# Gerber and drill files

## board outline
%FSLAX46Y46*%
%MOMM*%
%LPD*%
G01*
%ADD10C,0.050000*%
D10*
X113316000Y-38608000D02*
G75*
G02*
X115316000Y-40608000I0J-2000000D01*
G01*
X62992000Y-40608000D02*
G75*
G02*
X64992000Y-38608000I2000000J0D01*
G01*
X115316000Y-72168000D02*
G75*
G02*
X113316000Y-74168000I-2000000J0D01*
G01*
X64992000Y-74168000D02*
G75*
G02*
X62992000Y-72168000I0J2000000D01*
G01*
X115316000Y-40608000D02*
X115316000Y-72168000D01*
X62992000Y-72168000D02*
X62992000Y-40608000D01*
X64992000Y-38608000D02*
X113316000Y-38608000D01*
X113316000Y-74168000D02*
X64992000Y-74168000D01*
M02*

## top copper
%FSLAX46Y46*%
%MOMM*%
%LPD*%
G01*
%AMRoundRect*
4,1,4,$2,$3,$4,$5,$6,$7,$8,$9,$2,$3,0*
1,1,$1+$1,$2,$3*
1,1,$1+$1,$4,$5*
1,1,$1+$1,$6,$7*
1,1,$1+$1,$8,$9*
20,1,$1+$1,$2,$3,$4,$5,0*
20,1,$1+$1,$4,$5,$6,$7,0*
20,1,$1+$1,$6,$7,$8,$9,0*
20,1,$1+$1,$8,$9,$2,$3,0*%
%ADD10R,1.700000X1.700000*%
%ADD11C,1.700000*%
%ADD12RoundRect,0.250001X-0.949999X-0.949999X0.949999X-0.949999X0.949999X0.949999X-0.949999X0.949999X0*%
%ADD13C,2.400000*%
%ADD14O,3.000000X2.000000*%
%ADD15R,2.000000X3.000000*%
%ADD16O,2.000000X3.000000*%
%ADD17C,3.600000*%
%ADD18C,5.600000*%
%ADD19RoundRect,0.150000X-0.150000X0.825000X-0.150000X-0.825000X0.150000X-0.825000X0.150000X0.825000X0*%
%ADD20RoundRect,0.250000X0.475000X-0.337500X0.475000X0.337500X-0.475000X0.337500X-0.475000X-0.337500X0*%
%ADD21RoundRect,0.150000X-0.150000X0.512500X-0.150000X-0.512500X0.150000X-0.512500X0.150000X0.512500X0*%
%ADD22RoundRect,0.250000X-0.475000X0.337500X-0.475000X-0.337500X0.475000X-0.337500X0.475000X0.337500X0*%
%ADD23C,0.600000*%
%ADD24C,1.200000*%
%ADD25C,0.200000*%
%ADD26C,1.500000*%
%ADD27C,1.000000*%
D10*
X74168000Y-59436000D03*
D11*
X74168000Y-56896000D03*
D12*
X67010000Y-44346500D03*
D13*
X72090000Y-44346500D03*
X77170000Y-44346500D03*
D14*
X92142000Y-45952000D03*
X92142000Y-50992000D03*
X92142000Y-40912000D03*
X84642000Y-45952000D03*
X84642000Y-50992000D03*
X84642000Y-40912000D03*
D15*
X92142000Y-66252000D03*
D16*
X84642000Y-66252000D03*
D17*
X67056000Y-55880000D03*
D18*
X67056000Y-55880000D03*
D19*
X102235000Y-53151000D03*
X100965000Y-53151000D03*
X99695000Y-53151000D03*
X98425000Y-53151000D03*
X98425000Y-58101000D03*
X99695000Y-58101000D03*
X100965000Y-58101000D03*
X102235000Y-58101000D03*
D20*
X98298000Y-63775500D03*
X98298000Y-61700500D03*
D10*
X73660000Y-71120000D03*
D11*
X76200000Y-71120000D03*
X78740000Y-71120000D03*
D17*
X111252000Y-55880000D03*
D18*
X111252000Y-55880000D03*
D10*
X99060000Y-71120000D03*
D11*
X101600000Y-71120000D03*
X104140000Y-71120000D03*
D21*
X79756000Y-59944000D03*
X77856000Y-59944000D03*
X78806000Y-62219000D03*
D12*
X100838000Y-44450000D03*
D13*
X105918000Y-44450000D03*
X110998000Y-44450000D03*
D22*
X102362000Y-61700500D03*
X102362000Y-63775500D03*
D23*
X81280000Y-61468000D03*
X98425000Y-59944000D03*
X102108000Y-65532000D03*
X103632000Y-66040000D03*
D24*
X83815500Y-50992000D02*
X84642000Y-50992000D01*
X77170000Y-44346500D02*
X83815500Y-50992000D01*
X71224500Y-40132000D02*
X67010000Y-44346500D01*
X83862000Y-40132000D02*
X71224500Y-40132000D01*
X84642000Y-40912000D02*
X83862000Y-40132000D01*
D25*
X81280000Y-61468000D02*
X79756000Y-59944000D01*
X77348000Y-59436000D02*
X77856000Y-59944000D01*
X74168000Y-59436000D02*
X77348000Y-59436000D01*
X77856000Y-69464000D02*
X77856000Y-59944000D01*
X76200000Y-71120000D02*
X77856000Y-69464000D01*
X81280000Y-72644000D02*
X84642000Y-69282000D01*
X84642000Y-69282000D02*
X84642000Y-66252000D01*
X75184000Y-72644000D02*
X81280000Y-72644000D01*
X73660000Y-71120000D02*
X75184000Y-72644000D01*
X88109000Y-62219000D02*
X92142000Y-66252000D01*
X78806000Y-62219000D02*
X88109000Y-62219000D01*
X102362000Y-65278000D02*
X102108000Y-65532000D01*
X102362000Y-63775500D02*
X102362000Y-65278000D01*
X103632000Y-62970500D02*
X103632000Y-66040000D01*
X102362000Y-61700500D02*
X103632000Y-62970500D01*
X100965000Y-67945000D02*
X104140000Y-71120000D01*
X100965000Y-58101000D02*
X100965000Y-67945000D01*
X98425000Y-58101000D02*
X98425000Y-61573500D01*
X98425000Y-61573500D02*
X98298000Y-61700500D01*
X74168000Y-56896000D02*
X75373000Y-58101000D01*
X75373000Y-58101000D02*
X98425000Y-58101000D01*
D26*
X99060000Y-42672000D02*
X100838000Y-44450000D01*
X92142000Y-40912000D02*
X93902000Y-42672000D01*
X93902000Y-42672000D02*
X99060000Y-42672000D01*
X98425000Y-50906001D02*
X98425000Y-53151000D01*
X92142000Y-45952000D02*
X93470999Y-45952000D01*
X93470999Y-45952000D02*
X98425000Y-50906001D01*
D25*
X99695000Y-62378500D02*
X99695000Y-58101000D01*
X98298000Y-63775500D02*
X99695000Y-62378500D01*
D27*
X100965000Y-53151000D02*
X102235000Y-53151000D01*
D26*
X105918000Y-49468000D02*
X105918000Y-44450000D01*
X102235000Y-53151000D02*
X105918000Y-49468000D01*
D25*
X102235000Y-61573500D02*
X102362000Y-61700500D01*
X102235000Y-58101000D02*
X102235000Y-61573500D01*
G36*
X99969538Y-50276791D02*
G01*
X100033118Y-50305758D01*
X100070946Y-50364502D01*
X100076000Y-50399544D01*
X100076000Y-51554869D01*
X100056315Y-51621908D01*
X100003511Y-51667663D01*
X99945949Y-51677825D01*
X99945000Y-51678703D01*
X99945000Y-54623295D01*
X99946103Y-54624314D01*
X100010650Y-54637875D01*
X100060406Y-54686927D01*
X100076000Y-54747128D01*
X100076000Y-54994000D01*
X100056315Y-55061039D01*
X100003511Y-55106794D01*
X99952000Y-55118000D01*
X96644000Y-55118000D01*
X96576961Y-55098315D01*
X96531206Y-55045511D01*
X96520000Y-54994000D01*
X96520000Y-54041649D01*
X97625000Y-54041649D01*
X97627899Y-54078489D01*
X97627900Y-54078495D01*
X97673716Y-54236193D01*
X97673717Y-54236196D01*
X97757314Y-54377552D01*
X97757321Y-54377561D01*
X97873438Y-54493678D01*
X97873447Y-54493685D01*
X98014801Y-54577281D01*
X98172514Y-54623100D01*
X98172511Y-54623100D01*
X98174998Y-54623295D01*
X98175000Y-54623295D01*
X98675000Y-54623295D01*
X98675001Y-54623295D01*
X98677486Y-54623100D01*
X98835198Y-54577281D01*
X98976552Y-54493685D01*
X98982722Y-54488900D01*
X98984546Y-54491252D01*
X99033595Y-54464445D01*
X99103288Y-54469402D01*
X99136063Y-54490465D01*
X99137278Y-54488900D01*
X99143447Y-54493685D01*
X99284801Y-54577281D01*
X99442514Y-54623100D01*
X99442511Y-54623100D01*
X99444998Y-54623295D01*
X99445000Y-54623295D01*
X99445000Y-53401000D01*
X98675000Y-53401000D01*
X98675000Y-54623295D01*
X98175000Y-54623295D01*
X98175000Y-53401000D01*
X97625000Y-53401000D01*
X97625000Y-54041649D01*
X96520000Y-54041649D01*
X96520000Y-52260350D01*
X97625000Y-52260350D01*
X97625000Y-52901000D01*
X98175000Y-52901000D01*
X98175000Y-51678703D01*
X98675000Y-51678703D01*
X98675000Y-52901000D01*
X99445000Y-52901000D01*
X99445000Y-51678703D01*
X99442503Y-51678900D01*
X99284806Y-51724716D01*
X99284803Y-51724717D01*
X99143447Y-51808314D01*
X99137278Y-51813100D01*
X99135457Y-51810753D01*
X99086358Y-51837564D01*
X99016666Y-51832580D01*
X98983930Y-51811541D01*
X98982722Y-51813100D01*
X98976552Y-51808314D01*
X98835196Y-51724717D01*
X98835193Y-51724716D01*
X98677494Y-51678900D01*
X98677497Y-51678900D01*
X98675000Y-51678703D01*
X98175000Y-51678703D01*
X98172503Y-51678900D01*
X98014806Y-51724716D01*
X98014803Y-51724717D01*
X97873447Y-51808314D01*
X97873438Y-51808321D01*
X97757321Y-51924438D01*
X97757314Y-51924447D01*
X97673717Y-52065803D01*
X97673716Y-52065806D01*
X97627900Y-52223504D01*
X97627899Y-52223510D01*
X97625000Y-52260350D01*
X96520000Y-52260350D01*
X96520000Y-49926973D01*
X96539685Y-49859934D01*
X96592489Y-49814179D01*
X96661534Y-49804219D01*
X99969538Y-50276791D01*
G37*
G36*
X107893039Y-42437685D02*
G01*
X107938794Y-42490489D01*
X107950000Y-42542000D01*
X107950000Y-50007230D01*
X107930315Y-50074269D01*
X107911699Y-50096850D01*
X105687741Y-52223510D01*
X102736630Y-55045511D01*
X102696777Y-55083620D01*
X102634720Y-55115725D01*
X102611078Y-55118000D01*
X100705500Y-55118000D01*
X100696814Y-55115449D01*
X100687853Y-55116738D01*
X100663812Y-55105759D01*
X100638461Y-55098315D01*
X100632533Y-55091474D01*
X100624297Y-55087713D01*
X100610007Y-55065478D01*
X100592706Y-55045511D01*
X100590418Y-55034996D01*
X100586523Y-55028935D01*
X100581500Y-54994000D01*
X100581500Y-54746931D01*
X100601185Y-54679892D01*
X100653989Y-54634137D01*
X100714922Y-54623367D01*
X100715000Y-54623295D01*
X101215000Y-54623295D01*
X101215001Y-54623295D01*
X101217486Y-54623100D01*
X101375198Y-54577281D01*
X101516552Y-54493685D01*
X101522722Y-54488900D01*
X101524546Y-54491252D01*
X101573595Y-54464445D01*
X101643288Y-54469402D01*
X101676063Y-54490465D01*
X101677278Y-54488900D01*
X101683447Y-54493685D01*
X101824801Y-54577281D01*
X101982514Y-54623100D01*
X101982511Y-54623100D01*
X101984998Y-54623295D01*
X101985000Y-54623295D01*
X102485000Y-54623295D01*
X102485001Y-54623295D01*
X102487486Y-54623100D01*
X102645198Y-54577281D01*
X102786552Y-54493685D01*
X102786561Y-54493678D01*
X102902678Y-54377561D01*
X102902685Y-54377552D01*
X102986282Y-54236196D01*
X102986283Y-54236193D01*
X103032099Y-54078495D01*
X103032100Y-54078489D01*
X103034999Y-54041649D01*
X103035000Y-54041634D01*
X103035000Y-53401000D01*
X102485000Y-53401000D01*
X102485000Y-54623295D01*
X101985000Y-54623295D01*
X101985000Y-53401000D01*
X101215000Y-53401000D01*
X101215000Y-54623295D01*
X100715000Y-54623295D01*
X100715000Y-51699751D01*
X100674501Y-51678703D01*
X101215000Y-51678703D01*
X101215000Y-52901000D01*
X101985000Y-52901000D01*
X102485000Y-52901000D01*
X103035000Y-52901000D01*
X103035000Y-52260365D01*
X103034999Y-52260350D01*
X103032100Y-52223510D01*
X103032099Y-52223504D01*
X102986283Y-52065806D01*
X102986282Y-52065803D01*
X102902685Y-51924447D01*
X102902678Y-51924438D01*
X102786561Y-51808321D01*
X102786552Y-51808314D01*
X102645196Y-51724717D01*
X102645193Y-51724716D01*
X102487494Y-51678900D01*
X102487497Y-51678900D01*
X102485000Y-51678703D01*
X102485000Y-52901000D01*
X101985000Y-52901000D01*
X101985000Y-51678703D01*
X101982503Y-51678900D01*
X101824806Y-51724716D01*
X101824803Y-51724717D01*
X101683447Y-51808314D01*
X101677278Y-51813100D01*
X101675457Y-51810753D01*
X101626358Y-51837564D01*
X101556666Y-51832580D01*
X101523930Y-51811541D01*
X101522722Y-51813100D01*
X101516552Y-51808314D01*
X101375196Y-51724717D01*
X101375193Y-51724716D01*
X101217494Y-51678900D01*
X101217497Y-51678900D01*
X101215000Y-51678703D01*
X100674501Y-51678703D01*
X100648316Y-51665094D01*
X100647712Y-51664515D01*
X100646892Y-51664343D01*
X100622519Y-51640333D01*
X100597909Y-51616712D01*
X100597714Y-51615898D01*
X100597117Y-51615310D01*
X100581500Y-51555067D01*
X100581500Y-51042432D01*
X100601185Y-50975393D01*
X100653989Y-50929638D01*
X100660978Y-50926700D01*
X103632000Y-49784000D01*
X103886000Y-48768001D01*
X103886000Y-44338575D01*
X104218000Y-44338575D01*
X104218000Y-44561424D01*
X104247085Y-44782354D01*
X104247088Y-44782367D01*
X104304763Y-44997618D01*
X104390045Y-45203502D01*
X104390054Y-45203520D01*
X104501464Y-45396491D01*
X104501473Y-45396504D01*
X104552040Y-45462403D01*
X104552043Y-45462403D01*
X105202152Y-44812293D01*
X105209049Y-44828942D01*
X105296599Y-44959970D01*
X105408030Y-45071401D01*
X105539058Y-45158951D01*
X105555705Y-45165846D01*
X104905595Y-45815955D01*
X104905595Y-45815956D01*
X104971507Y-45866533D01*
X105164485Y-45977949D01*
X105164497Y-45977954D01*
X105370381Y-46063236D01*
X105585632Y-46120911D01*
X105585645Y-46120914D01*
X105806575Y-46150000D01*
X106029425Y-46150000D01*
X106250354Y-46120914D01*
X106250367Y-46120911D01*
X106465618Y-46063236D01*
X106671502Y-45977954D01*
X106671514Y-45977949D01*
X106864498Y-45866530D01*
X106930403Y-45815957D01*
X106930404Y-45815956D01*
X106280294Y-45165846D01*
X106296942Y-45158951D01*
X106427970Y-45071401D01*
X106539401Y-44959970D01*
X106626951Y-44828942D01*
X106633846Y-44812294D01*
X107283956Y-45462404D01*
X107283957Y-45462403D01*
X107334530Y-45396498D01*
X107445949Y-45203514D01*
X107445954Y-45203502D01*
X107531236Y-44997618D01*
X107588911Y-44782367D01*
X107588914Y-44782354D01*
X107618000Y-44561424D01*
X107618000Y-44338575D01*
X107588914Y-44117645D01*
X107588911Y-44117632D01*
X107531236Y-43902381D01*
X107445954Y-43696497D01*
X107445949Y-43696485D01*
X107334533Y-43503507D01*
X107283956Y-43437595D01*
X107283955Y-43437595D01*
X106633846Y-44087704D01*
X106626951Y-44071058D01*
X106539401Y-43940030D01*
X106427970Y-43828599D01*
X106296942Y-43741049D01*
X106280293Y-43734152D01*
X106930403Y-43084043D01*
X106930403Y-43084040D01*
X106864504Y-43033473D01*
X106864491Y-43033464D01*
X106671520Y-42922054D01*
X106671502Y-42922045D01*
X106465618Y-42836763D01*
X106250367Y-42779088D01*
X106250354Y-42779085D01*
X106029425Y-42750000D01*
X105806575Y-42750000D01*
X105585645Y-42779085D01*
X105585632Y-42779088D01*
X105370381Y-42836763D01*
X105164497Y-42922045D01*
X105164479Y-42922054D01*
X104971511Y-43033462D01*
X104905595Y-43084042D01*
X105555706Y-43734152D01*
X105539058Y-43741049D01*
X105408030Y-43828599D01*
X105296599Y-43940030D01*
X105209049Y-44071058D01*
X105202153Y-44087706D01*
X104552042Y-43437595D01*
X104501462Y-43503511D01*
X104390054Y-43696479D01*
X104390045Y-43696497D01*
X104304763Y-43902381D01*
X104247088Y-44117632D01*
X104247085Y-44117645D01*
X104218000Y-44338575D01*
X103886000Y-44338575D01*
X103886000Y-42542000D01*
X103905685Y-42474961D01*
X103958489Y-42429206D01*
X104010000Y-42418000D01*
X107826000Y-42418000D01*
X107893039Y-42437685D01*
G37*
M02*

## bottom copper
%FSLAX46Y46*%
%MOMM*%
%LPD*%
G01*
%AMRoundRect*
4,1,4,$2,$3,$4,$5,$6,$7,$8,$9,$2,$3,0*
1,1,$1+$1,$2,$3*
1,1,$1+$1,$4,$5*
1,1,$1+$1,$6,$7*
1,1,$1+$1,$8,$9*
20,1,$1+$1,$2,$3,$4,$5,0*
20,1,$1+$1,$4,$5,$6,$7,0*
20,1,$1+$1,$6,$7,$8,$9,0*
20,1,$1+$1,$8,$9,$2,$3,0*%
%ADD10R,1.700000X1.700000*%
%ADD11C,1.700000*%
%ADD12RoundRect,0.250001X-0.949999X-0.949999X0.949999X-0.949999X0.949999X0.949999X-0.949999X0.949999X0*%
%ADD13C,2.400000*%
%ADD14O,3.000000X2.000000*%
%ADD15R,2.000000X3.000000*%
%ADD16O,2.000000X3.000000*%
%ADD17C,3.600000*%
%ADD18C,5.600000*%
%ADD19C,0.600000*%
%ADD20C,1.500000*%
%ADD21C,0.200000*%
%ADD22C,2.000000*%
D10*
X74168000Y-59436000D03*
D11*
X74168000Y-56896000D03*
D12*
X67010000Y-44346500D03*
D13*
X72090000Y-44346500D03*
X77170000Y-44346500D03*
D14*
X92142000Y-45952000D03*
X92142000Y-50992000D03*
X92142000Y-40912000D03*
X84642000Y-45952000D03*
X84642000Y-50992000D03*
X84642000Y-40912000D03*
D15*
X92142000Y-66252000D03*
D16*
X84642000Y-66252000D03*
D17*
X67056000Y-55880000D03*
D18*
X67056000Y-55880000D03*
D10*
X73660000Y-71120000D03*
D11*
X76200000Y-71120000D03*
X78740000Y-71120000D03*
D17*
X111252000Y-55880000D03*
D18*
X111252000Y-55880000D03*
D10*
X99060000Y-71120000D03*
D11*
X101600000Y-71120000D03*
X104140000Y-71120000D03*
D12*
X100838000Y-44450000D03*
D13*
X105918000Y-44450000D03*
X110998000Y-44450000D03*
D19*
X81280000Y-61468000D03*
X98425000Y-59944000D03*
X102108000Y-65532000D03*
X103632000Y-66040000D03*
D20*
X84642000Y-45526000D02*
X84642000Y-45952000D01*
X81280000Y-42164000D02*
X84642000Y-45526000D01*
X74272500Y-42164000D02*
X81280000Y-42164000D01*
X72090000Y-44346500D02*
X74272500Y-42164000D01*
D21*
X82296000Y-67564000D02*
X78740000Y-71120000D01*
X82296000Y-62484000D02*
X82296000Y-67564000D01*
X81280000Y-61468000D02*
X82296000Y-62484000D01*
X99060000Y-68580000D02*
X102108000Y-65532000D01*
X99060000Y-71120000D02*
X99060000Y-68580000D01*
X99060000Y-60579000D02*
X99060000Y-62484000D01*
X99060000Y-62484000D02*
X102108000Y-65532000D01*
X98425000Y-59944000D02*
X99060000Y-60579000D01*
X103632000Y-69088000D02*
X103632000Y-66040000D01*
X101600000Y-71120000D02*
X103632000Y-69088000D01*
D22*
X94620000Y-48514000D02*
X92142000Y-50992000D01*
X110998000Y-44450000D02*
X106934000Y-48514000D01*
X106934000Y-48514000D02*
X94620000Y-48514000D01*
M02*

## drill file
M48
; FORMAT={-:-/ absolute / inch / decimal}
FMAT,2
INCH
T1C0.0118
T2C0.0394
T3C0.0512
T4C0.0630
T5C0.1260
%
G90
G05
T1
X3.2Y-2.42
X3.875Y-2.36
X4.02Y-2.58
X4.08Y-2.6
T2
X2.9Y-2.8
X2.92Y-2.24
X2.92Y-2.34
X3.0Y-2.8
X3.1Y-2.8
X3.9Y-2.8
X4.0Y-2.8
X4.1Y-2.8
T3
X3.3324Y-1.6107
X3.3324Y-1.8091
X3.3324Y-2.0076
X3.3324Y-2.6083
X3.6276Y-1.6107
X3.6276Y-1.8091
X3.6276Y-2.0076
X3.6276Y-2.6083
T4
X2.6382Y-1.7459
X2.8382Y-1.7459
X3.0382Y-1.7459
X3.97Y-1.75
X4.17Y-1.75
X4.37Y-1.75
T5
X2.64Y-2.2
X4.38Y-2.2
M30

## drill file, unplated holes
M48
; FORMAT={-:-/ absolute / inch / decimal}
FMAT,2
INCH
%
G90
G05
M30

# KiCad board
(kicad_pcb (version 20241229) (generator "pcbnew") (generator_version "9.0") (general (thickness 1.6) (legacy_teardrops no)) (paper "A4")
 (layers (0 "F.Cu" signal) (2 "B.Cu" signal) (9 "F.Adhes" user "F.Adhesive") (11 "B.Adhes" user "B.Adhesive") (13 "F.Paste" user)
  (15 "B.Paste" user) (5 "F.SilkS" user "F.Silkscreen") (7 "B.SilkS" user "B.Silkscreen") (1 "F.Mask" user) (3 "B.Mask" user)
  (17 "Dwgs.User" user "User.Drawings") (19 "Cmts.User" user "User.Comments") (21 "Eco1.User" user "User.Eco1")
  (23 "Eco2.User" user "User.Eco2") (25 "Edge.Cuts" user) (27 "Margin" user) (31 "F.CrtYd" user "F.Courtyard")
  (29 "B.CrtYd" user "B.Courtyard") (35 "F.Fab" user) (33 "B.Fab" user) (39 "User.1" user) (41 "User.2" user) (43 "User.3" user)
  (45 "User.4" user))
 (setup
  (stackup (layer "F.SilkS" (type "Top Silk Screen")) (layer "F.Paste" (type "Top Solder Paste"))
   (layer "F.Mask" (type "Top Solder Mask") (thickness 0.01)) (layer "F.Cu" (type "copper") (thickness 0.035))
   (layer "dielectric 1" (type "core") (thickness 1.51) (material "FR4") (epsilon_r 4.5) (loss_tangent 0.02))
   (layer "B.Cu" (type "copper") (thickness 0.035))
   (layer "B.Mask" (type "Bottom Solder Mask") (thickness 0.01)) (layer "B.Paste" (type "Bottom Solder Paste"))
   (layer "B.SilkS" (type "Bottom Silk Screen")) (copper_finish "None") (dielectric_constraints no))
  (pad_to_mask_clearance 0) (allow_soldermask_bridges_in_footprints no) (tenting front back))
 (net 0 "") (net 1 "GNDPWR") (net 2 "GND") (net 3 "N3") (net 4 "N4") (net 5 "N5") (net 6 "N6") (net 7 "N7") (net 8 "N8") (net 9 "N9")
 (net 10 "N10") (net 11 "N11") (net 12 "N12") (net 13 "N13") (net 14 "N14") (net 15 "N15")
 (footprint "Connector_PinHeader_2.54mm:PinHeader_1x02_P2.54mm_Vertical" (layer "F.Cu") (at 74.168 59.436 180)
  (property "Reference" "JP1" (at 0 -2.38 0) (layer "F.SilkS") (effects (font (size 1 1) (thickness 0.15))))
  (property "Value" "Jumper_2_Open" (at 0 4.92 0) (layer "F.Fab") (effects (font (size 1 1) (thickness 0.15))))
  (pad "1" thru_hole rect (at 0 0 180) (size 1.7 1.7) (drill 1) (layers "*.Cu" "*.Mask") (remove_unused_layers no) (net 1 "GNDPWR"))
  (pad "2" thru_hole circle (at 0 2.54 180) (size 1.7 1.7) (drill 1) (layers "*.Cu" "*.Mask") (remove_unused_layers no) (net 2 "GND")))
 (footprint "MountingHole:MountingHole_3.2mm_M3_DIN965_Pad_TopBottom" (layer "F.Cu") (at 67.056 55.88)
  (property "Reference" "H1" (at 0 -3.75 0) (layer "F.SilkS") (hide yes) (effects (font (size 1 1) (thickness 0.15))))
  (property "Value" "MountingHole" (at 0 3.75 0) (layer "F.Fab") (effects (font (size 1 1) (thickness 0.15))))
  (pad "1" thru_hole circle (at 0 0) (size 3.6 3.6) (drill 3.2) (layers "*.Cu" "*.Mask") (remove_unused_layers no) (zone_connect 2))
  (pad "1" connect circle (at 0 0) (size 5.6 5.6) (layers "F.Cu" "F.Mask") (zone_connect 2))
  (pad "1" connect circle (at 0 0) (size 5.6 5.6) (layers "B.Cu" "B.Mask") (zone_connect 2)))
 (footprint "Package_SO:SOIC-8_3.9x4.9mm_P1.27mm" (layer "F.Cu") (at 100.33 55.626 -90)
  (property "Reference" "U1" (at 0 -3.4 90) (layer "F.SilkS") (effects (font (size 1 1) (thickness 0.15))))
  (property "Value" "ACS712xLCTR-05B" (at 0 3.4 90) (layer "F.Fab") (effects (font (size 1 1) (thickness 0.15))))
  (pad "1" smd roundrect (at -2.475 -1.905 270) (size 1.95 0.6) (layers "F.Cu" "F.Mask" "F.Paste") (roundrect_rratio 0.25) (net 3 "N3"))
  (pad "2" smd roundrect (at -2.475 -0.635 270) (size 1.95 0.6) (layers "F.Cu" "F.Mask" "F.Paste") (roundrect_rratio 0.25) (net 3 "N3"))
  (pad "3" smd roundrect (at -2.475 0.635 270) (size 1.95 0.6) (layers "F.Cu" "F.Mask" "F.Paste") (roundrect_rratio 0.25) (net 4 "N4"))
  (pad "4" smd roundrect (at -2.475 1.905 270) (size 1.95 0.6) (layers "F.Cu" "F.Mask" "F.Paste") (roundrect_rratio 0.25) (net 4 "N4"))
  (pad "5" smd roundrect (at 2.475 1.905 270) (size 1.95 0.6) (layers "F.Cu" "F.Mask" "F.Paste") (roundrect_rratio 0.25) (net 2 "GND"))
  (pad "6" smd roundrect (at 2.475 0.635 270) (size 1.95 0.6) (layers "F.Cu" "F.Mask" "F.Paste") (roundrect_rratio 0.25) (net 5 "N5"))
  (pad "7" smd roundrect (at 2.475 -0.635 270) (size 1.95 0.6) (layers "F.Cu" "F.Mask" "F.Paste") (roundrect_rratio 0.25) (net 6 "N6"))
  (pad "8" smd roundrect (at 2.475 -1.905 270) (size 1.95 0.6) (layers "F.Cu" "F.Mask" "F.Paste") (roundrect_rratio 0.25) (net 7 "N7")))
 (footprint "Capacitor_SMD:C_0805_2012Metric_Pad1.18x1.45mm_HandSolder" (layer "F.Cu") (at 98.298 62.738 90)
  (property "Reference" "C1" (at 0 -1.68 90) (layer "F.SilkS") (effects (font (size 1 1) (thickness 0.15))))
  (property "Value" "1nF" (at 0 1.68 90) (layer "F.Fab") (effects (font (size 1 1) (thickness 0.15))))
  (pad "1" smd roundrect (at -1.0375 0 90) (size 1.175 1.45) (layers "F.Cu" "F.Mask" "F.Paste") (roundrect_rratio 0.212766) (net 5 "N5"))
  (pad "2" smd roundrect (at 1.0375 0 90) (size 1.175 1.45) (layers "F.Cu" "F.Mask" "F.Paste") (roundrect_rratio 0.212766) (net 2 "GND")))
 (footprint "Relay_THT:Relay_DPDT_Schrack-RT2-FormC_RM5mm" (layer "F.Cu") (at 92.142 66.252 90)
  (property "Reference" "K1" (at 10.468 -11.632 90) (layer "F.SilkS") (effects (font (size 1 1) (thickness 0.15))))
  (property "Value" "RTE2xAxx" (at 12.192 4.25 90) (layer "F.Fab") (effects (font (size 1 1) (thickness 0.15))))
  (pad "11" thru_hole oval (at 20.3 0 270) (size 2 3) (drill 1.3) (layers "*.Cu" "*.Mask") (remove_unused_layers no) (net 4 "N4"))
  (pad "12" thru_hole oval (at 15.26 0 270) (size 2 3) (drill 1.3) (layers "*.Cu" "*.Mask") (remove_unused_layers no) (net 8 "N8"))
  (pad "14" thru_hole oval (at 25.34 0 270) (size 2 3) (drill 1.3) (layers "*.Cu" "*.Mask") (remove_unused_layers no) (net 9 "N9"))
  (pad "21" thru_hole oval (at 20.3 -7.5 270) (size 2 3) (drill 1.3) (layers "*.Cu" "*.Mask") (remove_unused_layers no) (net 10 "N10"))
  (pad "22" thru_hole oval (at 15.26 -7.5 270) (size 2 3) (drill 1.3) (layers "*.Cu" "*.Mask") (remove_unused_layers no) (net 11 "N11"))
  (pad "24" thru_hole oval (at 25.34 -7.5 270) (size 2 3) (drill 1.3) (layers "*.Cu" "*.Mask") (remove_unused_layers no) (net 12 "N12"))
  (pad "A1" thru_hole rect (at 0 0 270) (size 3 2) (drill 1.3) (layers "*.Cu" "*.Mask") (remove_unused_layers no) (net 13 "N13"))
  (pad "A2" thru_hole oval (at 0 -7.5 270) (size 3 2) (drill 1.3) (layers "*.Cu" "*.Mask") (remove_unused_layers no) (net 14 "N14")))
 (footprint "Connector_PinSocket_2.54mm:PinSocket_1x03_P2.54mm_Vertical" (layer "F.Cu") (at 73.66 71.12 90)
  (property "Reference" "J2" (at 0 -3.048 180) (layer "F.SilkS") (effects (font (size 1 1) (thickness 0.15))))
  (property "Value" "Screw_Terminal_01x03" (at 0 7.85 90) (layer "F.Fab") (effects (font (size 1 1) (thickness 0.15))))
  (pad "1" thru_hole rect (at 0 0 90) (size 1.7 1.7) (drill 1) (layers "*.Cu" "*.Mask") (remove_unused_layers no) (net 14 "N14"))
  (pad "2" thru_hole circle (at 0 2.54 90) (size 1.7 1.7) (drill 1) (layers "*.Cu" "*.Mask") (remove_unused_layers no) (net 1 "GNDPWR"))
  (pad "3" thru_hole circle (at 0 5.08 90) (size 1.7 1.7) (drill 1) (layers "*.Cu" "*.Mask") (remove_unused_layers no) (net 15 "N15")))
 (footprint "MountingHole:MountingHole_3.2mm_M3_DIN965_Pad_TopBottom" (layer "F.Cu") (at 111.252 55.88)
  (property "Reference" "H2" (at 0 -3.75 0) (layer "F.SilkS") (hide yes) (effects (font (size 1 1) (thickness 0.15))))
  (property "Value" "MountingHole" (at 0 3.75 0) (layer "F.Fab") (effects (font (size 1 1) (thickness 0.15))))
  (pad "1" thru_hole circle (at 0 0) (size 3.6 3.6) (drill 3.2) (layers "*.Cu" "*.Mask") (remove_unused_layers no) (zone_connect 2))
  (pad "1" connect circle (at 0 0) (size 5.6 5.6) (layers "F.Cu" "F.Mask") (zone_connect 2))
  (pad "1" connect circle (at 0 0) (size 5.6 5.6) (layers "B.Cu" "B.Mask") (zone_connect 2)))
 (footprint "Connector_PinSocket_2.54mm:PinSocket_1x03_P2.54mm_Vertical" (layer "F.Cu") (at 99.06 71.12 90)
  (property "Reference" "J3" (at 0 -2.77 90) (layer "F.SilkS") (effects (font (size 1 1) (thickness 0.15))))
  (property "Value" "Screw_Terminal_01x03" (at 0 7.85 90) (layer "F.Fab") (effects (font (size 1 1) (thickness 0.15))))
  (pad "1" thru_hole rect (at 0 0 90) (size 1.7 1.7) (drill 1) (layers "*.Cu" "*.Mask") (remove_unused_layers no) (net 2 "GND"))
  (pad "2" thru_hole circle (at 0 2.54 90) (size 1.7 1.7) (drill 1) (layers "*.Cu" "*.Mask") (remove_unused_layers no) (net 7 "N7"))
  (pad "3" thru_hole circle (at 0 5.08 90) (size 1.7 1.7) (drill 1) (layers "*.Cu" "*.Mask") (remove_unused_layers no) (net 6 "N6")))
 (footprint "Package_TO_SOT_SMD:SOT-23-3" (layer "F.Cu") (at 78.806 61.0815 -90)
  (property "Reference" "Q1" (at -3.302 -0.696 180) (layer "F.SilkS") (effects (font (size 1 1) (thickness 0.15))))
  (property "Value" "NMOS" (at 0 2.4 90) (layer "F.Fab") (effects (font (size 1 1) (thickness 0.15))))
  (pad "1" smd roundrect (at -1.1375 -0.95 270) (size 1.325 0.6) (layers "F.Cu" "F.Mask" "F.Paste") (roundrect_rratio 0.25) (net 15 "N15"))
  (pad "2" smd roundrect (at -1.1375 0.95 270) (size 1.325 0.6) (layers "F.Cu" "F.Mask" "F.Paste") (roundrect_rratio 0.25) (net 1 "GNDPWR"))
  (pad "3" smd roundrect (at 1.1375 0 270) (size 1.325 0.6) (layers "F.Cu" "F.Mask" "F.Paste") (roundrect_rratio 0.25) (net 13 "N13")))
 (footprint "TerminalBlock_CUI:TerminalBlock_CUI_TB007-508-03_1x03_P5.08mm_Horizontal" (layer "F.Cu") (at 67.01 44.3465)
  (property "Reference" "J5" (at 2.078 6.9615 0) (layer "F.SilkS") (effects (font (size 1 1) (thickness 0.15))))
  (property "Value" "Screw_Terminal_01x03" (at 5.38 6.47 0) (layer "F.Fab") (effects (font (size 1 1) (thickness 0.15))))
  (pad "1" thru_hole roundrect (at 0 0) (size 2.4 2.4) (drill 1.6) (layers "*.Cu" "*.Mask") (remove_unused_layers no)
   (roundrect_rratio 0.104167) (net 12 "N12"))
  (pad "2" thru_hole circle (at 5.08 0) (size 2.4 2.4) (drill 1.6) (layers "*.Cu" "*.Mask") (remove_unused_layers no) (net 10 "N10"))
  (pad "3" thru_hole circle (at 10.16 0) (size 2.4 2.4) (drill 1.6) (layers "*.Cu" "*.Mask") (remove_unused_layers no) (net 11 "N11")))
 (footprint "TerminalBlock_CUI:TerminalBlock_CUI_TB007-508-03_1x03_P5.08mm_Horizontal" (layer "F.Cu") (at 100.838 44.45)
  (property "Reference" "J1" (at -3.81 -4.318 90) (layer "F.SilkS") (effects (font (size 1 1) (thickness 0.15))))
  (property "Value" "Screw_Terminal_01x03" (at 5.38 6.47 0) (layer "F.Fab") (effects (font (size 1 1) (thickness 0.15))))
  (pad "1" thru_hole roundrect (at 0 0) (size 2.4 2.4) (drill 1.6) (layers "*.Cu" "*.Mask") (remove_unused_layers no)
   (roundrect_rratio 0.104167) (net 9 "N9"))
  (pad "2" thru_hole circle (at 5.08 0) (size 2.4 2.4) (drill 1.6) (layers "*.Cu" "*.Mask") (remove_unused_layers no) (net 3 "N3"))
  (pad "3" thru_hole circle (at 10.16 0) (size 2.4 2.4) (drill 1.6) (layers "*.Cu" "*.Mask") (remove_unused_layers no) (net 8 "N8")))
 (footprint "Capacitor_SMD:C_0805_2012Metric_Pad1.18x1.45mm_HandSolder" (layer "F.Cu") (at 102.362 62.738 -90)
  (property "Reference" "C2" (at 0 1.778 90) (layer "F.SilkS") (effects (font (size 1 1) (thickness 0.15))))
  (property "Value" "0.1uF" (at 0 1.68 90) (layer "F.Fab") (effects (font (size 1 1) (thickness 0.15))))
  (pad "1" smd roundrect (at -1.0375 0 270) (size 1.175 1.45) (layers "F.Cu" "F.Mask" "F.Paste") (roundrect_rratio 0.212766) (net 7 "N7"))
  (pad "2" smd roundrect (at 1.0375 0 270) (size 1.175 1.45) (layers "F.Cu" "F.Mask" "F.Paste") (roundrect_rratio 0.212766) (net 2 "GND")))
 (gr_line (start 115.316 40.608) (end 115.316 72.168) (stroke (width 0.05) (type default)) (layer "Edge.Cuts"))
 (gr_arc (start 62.992 40.608) (mid 63.577786 39.193786) (end 64.992 38.608) (stroke (width 0.05) (type default)) (layer "Edge.Cuts"))
 (gr_arc (start 113.316 38.608) (mid 114.730214 39.193786) (end 115.316 40.608) (stroke (width 0.05) (type default)) (layer "Edge.Cuts"))
 (gr_line (start 113.316 74.168) (end 64.992 74.168) (stroke (width 0.05) (type default)) (layer "Edge.Cuts"))
 (gr_line (start 64.992 38.608) (end 113.316 38.608) (stroke (width 0.05) (type default)) (layer "Edge.Cuts"))
 (gr_line (start 62.992 72.168) (end 62.992 40.608) (stroke (width 0.05) (type default)) (layer "Edge.Cuts"))
 (gr_arc (start 115.316 72.168) (mid 114.730214 73.582214) (end 113.316 74.168) (stroke (width 0.05) (type default)) (layer "Edge.Cuts"))
 (gr_arc (start 64.992 74.168) (mid 63.577786 73.582214) (end 62.992 72.168) (stroke (width 0.05) (type default)) (layer "Edge.Cuts"))
 (segment (start 99.695 62.3785) (end 99.695 58.101) (width 0.2) (layer "F.Cu") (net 5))
 (segment (start 98.298 63.7755) (end 99.695 62.3785) (width 0.2) (layer "F.Cu") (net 5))
 (segment (start 102.362 65.278) (end 102.108 65.532) (width 0.2) (layer "F.Cu") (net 2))
 (segment (start 98.425 58.101) (end 98.425 61.5735) (width 0.2) (layer "F.Cu") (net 2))
 (segment (start 75.373 58.101) (end 98.425 58.101) (width 0.2) (layer "F.Cu") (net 2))
 (segment (start 74.168 56.896) (end 75.373 58.101) (width 0.2) (layer "F.Cu") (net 2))
 (segment (start 102.362 63.7755) (end 102.362 65.278) (width 0.2) (layer "F.Cu") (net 2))
 (segment (start 98.425 61.5735) (end 98.298 61.7005) (width 0.2) (layer "F.Cu") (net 2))
 (via (at 98.425 59.944) (size 0.6) (drill 0.3) (layers "F.Cu" "B.Cu") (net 2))
 (via (at 102.108 65.532) (size 0.6) (drill 0.3) (layers "F.Cu" "B.Cu") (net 2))
 (segment (start 99.06 62.484) (end 102.108 65.532) (width 0.2) (layer "B.Cu") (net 2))
 (segment (start 99.06 60.579) (end 99.06 62.484) (width 0.2) (layer "B.Cu") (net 2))
 (segment (start 99.06 68.58) (end 102.108 65.532) (width 0.2) (layer "B.Cu") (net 2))
 (segment (start 98.425 59.944) (end 99.06 60.579) (width 0.2) (layer "B.Cu") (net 2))
 (segment (start 99.06 71.12) (end 99.06 68.58) (width 0.2) (layer "B.Cu") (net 2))
 (segment (start 100.965 53.151) (end 102.235 53.151) (width 1) (layer "F.Cu") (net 3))
 (segment (start 105.918 49.468) (end 105.918 44.45) (width 1.5) (layer "F.Cu") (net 3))
 (segment (start 102.235 53.151) (end 105.918 49.468) (width 1.5) (layer "F.Cu") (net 3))
 (segment (start 92.142 40.912) (end 93.902 42.672) (width 1.5) (layer "F.Cu") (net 9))
 (segment (start 99.06 42.672) (end 100.838 44.45) (width 1.5) (layer "F.Cu") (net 9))
 (segment (start 93.902 42.672) (end 99.06 42.672) (width 1.5) (layer "F.Cu") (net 9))
 (segment (start 75.184 72.644) (end 81.28 72.644) (width 0.2) (layer "F.Cu") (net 14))
 (segment (start 81.28 72.644) (end 84.642 69.282) (width 0.2) (layer "F.Cu") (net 14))
 (segment (start 73.66 71.12) (end 75.184 72.644) (width 0.2) (layer "F.Cu") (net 14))
 (segment (start 84.642 69.282) (end 84.642 66.252) (width 0.2) (layer "F.Cu") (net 14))
 (segment (start 81.28 61.468) (end 79.756 59.944) (width 0.2) (layer "F.Cu") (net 15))
 (via (at 81.28 61.468) (size 0.6) (drill 0.3) (layers "F.Cu" "B.Cu") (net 15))
 (segment (start 81.28 61.468) (end 82.296 62.484) (width 0.2) (layer "B.Cu") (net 15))
 (segment (start 82.296 67.564) (end 78.74 71.12) (width 0.2) (layer "B.Cu") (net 15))
 (segment (start 82.296 62.484) (end 82.296 67.564) (width 0.2) (layer "B.Cu") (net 15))
 (segment (start 77.856 69.464) (end 77.856 59.944) (width 0.2) (layer "F.Cu") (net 1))
 (segment (start 76.2 71.12) (end 77.856 69.464) (width 0.2) (layer "F.Cu") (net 1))
 (segment (start 74.168 59.436) (end 77.348 59.436) (width 0.2) (layer "F.Cu") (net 1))
 (segment (start 77.348 59.436) (end 77.856 59.944) (width 0.2) (layer "F.Cu") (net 1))
 (segment (start 88.109 62.219) (end 92.142 66.252) (width 0.2) (layer "F.Cu") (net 13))
 (segment (start 78.806 62.219) (end 88.109 62.219) (width 0.2) (layer "F.Cu") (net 13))
 (segment (start 106.934 48.514) (end 94.62 48.514) (width 2) (layer "B.Cu") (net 8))
 (segment (start 110.998 44.45) (end 106.934 48.514) (width 2) (layer "B.Cu") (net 8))
 (segment (start 94.62 48.514) (end 92.142 50.992) (width 2) (layer "B.Cu") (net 8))
 (segment (start 103.632 62.9705) (end 103.632 66.04) (width 0.2) (layer "F.Cu") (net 7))
 (segment (start 102.362 61.7005) (end 103.632 62.9705) (width 0.2) (layer "F.Cu") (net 7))
 (segment (start 102.235 61.5735) (end 102.362 61.7005) (width 0.2) (layer "F.Cu") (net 7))
 (segment (start 102.235 58.101) (end 102.235 61.5735) (width 0.2) (layer "F.Cu") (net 7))
 (via (at 103.632 66.04) (size 0.6) (drill 0.3) (layers "F.Cu" "B.Cu") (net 7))
 (segment (start 103.632 69.088) (end 103.632 66.04) (width 0.2) (layer "B.Cu") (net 7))
 (segment (start 101.6 71.12) (end 103.632 69.088) (width 0.2) (layer "B.Cu") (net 7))
 (segment (start 100.965 67.945) (end 104.14 71.12) (width 0.2) (layer "F.Cu") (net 6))
 (segment (start 100.965 58.101) (end 100.965 67.945) (width 0.2) (layer "F.Cu") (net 6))
 (segment (start 92.142 45.952) (end 93.470999 45.952) (width 1.5) (layer "F.Cu") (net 4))
 (segment (start 93.470999 45.952) (end 98.425 50.906001) (width 1.5) (layer "F.Cu") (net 4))
 (segment (start 98.425 50.906001) (end 98.425 53.151) (width 1.5) (layer "F.Cu") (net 4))
 (segment (start 84.642 40.912) (end 83.862 40.132) (width 1.2) (layer "F.Cu") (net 12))
 (segment (start 71.2245 40.132) (end 67.01 44.3465) (width 1.2) (layer "F.Cu") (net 12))
 (segment (start 83.862 40.132) (end 71.2245 40.132) (width 1.2) (layer "F.Cu") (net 12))
 (segment (start 83.8155 50.992) (end 84.642 50.992) (width 1.2) (layer "F.Cu") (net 11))
 (segment (start 77.17 44.3465) (end 83.8155 50.992) (width 1.2) (layer "F.Cu") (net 11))
 (segment (start 81.28 42.164) (end 84.642 45.526) (width 1.5) (layer "B.Cu") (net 10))
 (segment (start 74.2725 42.164) (end 81.28 42.164) (width 1.5) (layer "B.Cu") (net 10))
 (segment (start 72.09 44.3465) (end 74.2725 42.164) (width 1.5) (layer "B.Cu") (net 10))
 (segment (start 84.642 45.526) (end 84.642 45.952) (width 1.5) (layer "B.Cu") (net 10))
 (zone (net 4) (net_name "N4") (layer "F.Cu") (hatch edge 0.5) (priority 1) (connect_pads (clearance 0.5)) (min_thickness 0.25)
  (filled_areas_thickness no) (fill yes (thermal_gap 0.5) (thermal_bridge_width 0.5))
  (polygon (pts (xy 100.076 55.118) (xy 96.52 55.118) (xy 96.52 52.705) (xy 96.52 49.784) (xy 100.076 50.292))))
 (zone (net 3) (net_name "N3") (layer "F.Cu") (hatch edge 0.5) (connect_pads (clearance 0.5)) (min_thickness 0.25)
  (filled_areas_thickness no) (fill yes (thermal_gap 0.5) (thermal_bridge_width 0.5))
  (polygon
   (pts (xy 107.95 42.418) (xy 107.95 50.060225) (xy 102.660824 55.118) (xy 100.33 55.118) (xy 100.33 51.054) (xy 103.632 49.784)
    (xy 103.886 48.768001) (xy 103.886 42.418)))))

